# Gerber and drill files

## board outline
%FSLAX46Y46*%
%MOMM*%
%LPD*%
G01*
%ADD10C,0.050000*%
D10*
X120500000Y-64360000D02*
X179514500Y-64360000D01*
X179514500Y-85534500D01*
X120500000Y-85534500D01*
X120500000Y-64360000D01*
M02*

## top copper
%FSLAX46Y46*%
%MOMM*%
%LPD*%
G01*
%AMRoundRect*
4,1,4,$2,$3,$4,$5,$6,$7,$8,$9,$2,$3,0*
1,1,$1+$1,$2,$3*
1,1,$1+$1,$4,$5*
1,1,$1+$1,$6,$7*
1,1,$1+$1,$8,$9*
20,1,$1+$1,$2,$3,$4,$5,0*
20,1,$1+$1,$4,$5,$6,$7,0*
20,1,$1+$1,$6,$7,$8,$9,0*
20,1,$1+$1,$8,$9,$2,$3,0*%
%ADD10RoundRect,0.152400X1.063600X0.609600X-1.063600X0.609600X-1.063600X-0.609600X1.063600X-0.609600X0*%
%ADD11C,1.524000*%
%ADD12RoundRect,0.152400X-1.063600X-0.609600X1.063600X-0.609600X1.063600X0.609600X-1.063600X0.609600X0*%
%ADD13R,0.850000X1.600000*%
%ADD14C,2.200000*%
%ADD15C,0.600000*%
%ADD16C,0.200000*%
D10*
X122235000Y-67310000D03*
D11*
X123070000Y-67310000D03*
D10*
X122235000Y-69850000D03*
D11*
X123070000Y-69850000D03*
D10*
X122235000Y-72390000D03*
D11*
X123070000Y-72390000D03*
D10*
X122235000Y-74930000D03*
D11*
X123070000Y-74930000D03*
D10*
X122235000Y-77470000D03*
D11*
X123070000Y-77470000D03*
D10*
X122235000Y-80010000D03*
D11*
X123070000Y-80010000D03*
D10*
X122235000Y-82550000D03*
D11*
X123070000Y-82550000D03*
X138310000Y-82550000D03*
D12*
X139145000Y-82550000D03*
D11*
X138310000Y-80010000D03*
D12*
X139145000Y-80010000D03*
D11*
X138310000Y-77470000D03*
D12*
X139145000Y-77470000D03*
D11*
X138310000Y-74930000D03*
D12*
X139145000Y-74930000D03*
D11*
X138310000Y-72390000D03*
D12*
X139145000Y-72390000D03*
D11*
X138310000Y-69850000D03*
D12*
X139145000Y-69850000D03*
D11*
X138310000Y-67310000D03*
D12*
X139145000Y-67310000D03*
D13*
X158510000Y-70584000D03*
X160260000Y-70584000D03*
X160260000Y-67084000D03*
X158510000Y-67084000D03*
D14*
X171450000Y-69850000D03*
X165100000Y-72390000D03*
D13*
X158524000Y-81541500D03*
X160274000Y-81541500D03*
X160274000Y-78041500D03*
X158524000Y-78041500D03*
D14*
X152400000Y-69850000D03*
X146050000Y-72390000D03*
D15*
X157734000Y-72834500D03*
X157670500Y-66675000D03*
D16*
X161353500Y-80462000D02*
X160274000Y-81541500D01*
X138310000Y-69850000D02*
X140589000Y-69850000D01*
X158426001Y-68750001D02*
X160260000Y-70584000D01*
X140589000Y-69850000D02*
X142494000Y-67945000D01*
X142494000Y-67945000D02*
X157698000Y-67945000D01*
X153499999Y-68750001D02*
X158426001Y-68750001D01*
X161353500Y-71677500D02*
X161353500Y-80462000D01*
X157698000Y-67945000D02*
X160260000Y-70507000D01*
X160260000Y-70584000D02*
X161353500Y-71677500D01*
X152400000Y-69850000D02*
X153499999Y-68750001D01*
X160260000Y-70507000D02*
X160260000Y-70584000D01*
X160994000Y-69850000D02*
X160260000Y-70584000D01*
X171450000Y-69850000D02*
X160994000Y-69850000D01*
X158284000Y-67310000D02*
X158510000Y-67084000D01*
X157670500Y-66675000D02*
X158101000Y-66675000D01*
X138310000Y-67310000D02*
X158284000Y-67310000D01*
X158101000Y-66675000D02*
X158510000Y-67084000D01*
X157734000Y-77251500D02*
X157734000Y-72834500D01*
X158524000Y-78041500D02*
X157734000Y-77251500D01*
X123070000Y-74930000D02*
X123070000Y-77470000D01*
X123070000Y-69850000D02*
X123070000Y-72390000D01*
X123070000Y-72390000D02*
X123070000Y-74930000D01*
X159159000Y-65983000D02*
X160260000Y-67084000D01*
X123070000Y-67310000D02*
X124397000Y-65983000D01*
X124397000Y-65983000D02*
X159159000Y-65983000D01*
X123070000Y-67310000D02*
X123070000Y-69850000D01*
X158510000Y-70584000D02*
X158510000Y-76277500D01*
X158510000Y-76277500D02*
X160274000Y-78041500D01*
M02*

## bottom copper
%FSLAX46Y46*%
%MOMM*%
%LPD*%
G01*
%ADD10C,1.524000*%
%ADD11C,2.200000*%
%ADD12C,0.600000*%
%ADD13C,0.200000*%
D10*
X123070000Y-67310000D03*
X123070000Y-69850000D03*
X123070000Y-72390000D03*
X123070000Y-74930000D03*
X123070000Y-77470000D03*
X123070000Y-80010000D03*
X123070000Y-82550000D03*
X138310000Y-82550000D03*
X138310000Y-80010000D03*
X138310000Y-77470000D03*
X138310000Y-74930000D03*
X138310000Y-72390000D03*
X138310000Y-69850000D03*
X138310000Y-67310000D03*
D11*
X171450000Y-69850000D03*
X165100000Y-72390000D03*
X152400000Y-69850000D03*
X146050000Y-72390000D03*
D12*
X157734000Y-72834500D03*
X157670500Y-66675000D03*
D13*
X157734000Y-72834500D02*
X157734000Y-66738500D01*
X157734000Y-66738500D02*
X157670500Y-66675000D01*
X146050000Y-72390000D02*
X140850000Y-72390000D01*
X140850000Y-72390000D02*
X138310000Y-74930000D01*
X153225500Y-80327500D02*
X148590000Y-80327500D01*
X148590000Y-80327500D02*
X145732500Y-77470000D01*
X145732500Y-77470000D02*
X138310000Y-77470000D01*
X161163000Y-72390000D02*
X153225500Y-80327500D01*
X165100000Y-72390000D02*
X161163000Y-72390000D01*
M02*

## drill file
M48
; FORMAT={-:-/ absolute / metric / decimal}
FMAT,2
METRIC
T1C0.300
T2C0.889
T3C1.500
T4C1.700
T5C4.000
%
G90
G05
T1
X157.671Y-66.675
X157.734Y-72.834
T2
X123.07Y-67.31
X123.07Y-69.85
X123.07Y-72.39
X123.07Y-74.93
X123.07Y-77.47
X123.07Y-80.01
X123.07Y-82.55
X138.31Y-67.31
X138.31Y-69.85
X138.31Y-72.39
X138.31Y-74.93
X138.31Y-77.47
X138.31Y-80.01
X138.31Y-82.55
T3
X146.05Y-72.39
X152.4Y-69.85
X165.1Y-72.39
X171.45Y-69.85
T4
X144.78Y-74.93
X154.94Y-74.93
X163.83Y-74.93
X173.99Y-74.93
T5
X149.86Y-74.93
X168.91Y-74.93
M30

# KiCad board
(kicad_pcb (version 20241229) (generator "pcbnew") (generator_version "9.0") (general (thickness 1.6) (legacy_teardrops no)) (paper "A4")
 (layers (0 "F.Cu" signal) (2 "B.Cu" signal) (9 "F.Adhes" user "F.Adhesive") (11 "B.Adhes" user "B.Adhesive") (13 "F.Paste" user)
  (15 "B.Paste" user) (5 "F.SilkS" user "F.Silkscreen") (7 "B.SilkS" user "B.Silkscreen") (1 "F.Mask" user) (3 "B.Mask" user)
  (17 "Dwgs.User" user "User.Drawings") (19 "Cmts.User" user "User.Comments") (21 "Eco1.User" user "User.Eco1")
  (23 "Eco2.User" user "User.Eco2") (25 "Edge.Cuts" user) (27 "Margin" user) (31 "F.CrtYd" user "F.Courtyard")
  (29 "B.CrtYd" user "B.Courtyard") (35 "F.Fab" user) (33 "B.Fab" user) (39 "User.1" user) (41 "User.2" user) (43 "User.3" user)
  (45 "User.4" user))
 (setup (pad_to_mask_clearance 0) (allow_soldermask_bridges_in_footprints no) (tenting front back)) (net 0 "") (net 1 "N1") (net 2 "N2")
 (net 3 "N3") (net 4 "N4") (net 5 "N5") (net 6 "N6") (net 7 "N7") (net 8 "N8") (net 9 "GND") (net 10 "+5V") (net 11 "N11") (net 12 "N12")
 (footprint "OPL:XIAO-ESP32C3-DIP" (layer "F.Cu") (at 130.81 74.93)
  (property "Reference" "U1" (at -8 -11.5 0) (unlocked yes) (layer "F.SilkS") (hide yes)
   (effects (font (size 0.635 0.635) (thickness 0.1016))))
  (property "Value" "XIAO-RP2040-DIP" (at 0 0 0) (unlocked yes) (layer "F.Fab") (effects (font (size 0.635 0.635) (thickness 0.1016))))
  (pad "1" smd roundrect (at -8.575 -7.62 180) (size 2.432 1.524) (layers "F.Cu" "F.Mask") (roundrect_rratio 0.1) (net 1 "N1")
   (thermal_bridge_angle 45))
  (pad "1" thru_hole circle (at -7.74 -7.62 180) (size 1.524 1.524) (drill 0.889) (layers "*.Cu" "*.Mask") (remove_unused_layers no)
   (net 1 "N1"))
  (pad "2" smd roundrect (at -8.575 -5.08 180) (size 2.432 1.524) (layers "F.Cu" "F.Mask") (roundrect_rratio 0.1) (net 1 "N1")
   (thermal_bridge_angle 45))
  (pad "2" thru_hole circle (at -7.74 -5.08 180) (size 1.524 1.524) (drill 0.889) (layers "*.Cu" "*.Mask") (remove_unused_layers no)
   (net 1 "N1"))
  (pad "3" smd roundrect (at -8.575 -2.54 180) (size 2.432 1.524) (layers "F.Cu" "F.Mask") (roundrect_rratio 0.1) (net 1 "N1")
   (thermal_bridge_angle 45))
  (pad "3" thru_hole circle (at -7.74 -2.54 180) (size 1.524 1.524) (drill 0.889) (layers "*.Cu" "*.Mask") (remove_unused_layers no)
   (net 1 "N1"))
  (pad "4" smd roundrect (at -8.575 0 180) (size 2.432 1.524) (layers "F.Cu" "F.Mask") (roundrect_rratio 0.1) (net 1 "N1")
   (thermal_bridge_angle 45))
  (pad "4" thru_hole circle (at -7.74 0 180) (size 1.524 1.524) (drill 0.889) (layers "*.Cu" "*.Mask") (remove_unused_layers no)
   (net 1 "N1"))
  (pad "5" smd roundrect (at -8.575 2.54 180) (size 2.432 1.524) (layers "F.Cu" "F.Mask") (roundrect_rratio 0.1) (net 1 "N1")
   (thermal_bridge_angle 45))
  (pad "5" thru_hole circle (at -7.74 2.54 180) (size 1.524 1.524) (drill 0.889) (layers "*.Cu" "*.Mask") (remove_unused_layers no)
   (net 1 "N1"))
  (pad "6" smd roundrect (at -8.575 5.08 180) (size 2.432 1.524) (layers "F.Cu" "F.Mask") (roundrect_rratio 0.1) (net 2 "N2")
   (thermal_bridge_angle 45))
  (pad "6" thru_hole circle (at -7.74 5.08 180) (size 1.524 1.524) (drill 0.889) (layers "*.Cu" "*.Mask") (remove_unused_layers no)
   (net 2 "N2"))
  (pad "7" smd roundrect (at -8.575 7.62 180) (size 2.432 1.524) (layers "F.Cu" "F.Mask") (roundrect_rratio 0.1) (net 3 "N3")
   (thermal_bridge_angle 45))
  (pad "7" thru_hole circle (at -7.74 7.62 180) (size 1.524 1.524) (drill 0.889) (layers "*.Cu" "*.Mask") (remove_unused_layers no)
   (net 3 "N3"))
  (pad "8" thru_hole circle (at 7.5 7.62) (size 1.524 1.524) (drill 0.889) (layers "*.Cu" "*.Mask") (remove_unused_layers no) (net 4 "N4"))
  (pad "8" smd roundrect (at 8.335 7.62) (size 2.432 1.524) (layers "F.Cu" "F.Mask") (roundrect_rratio 0.1) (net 4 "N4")
   (thermal_bridge_angle 45))
  (pad "9" thru_hole circle (at 7.5 5.08) (size 1.524 1.524) (drill 0.889) (layers "*.Cu" "*.Mask") (remove_unused_layers no) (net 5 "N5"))
  (pad "9" smd roundrect (at 8.335 5.08) (size 2.432 1.524) (layers "F.Cu" "F.Mask") (roundrect_rratio 0.1) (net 5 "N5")
   (thermal_bridge_angle 45))
  (pad "10" thru_hole circle (at 7.5 2.54) (size 1.524 1.524) (drill 0.889) (layers "*.Cu" "*.Mask") (remove_unused_layers no) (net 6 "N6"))
  (pad "10" smd roundrect (at 8.335 2.54) (size 2.432 1.524) (layers "F.Cu" "F.Mask") (roundrect_rratio 0.1) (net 6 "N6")
   (thermal_bridge_angle 45))
  (pad "11" thru_hole circle (at 7.5 0) (size 1.524 1.524) (drill 0.889) (layers "*.Cu" "*.Mask") (remove_unused_layers no) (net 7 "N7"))
  (pad "11" smd roundrect (at 8.335 0) (size 2.432 1.524) (layers "F.Cu" "F.Mask") (roundrect_rratio 0.1) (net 7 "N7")
   (thermal_bridge_angle 45))
  (pad "12" thru_hole circle (at 7.5 -2.54) (size 1.524 1.524) (drill 0.889) (layers "*.Cu" "*.Mask") (remove_unused_layers no) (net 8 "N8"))
  (pad "12" smd roundrect (at 8.335 -2.54) (size 2.432 1.524) (layers "F.Cu" "F.Mask") (roundrect_rratio 0.1) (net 8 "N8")
   (thermal_bridge_angle 45))
  (pad "13" thru_hole circle (at 7.5 -5.08) (size 1.524 1.524) (drill 0.889) (layers "*.Cu" "*.Mask") (remove_unused_layers no)
   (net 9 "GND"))
  (pad "13" smd roundrect (at 8.335 -5.08) (size 2.432 1.524) (layers "F.Cu" "F.Mask") (roundrect_rratio 0.1) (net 9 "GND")
   (thermal_bridge_angle 45))
  (pad "14" thru_hole circle (at 7.5 -7.62) (size 1.524 1.524) (drill 0.889) (layers "*.Cu" "*.Mask") (remove_unused_layers no)
   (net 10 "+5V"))
  (pad "14" smd roundrect (at 8.335 -7.62) (size 2.432 1.524) (layers "F.Cu" "F.Mask") (roundrect_rratio 0.1) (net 10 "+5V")
   (thermal_bridge_angle 45)))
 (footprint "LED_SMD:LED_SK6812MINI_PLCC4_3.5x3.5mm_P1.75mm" (layer "F.Cu") (at 159.385 68.834 90)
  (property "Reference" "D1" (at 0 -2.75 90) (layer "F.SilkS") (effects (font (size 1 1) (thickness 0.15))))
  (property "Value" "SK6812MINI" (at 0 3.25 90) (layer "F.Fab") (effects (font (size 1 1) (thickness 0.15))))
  (pad "1" smd rect (at -1.75 -0.875 90) (size 1.6 0.85) (layers "F.Cu" "F.Mask" "F.Paste") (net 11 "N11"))
  (pad "2" smd rect (at -1.75 0.875 90) (size 1.6 0.85) (layers "F.Cu" "F.Mask" "F.Paste") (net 9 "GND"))
  (pad "3" smd rect (at 1.75 0.875 90) (size 1.6 0.85) (layers "F.Cu" "F.Mask" "F.Paste") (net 1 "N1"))
  (pad "4" smd rect (at 1.75 -0.875 90) (size 1.6 0.85) (layers "F.Cu" "F.Mask" "F.Paste") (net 10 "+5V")))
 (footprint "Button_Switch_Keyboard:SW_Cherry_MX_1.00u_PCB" (layer "F.Cu") (at 171.45 69.85)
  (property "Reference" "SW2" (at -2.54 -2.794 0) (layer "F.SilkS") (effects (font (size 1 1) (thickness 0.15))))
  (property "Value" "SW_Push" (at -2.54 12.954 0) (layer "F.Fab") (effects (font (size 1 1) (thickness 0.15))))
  (pad "" np_thru_hole circle (at -7.62 5.08) (size 1.7 1.7) (drill 1.7) (layers "*.Cu" "*.Mask"))
  (pad "" np_thru_hole circle (at -2.54 5.08) (size 4 4) (drill 4) (layers "*.Cu" "*.Mask"))
  (pad "" np_thru_hole circle (at 2.54 5.08) (size 1.7 1.7) (drill 1.7) (layers "*.Cu" "*.Mask"))
  (pad "1" thru_hole circle (at 0 0) (size 2.2 2.2) (drill 1.5) (layers "*.Cu" "*.Mask") (remove_unused_layers no) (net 9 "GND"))
  (pad "2" thru_hole circle (at -6.35 2.54) (size 2.2 2.2) (drill 1.5) (layers "*.Cu" "*.Mask") (remove_unused_layers no) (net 6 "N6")))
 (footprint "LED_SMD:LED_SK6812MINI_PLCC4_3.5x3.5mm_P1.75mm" (layer "F.Cu") (at 159.399 79.7915 90)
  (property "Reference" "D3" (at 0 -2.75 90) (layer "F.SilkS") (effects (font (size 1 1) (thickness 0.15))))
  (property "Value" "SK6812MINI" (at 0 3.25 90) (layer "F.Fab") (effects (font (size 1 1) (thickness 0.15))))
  (pad "1" smd rect (at -1.75 -0.875 90) (size 1.6 0.85) (layers "F.Cu" "F.Mask" "F.Paste") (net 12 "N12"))
  (pad "2" smd rect (at -1.75 0.875 90) (size 1.6 0.85) (layers "F.Cu" "F.Mask" "F.Paste") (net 9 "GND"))
  (pad "3" smd rect (at 1.75 0.875 90) (size 1.6 0.85) (layers "F.Cu" "F.Mask" "F.Paste") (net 11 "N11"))
  (pad "4" smd rect (at 1.75 -0.875 90) (size 1.6 0.85) (layers "F.Cu" "F.Mask" "F.Paste") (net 10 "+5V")))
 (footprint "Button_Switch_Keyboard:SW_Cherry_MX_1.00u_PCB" (layer "F.Cu") (at 152.4 69.85)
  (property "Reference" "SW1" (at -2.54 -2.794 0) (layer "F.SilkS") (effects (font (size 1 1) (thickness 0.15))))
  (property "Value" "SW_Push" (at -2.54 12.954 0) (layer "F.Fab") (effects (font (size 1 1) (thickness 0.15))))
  (pad "" np_thru_hole circle (at -7.62 5.08) (size 1.7 1.7) (drill 1.7) (layers "*.Cu" "*.Mask"))
  (pad "" np_thru_hole circle (at -2.54 5.08) (size 4 4) (drill 4) (layers "*.Cu" "*.Mask"))
  (pad "" np_thru_hole circle (at 2.54 5.08) (size 1.7 1.7) (drill 1.7) (layers "*.Cu" "*.Mask"))
  (pad "1" thru_hole circle (at 0 0) (size 2.2 2.2) (drill 1.5) (layers "*.Cu" "*.Mask") (remove_unused_layers no) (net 9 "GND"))
  (pad "2" thru_hole circle (at -6.35 2.54) (size 2.2 2.2) (drill 1.5) (layers "*.Cu" "*.Mask") (remove_unused_layers no) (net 7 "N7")))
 (gr_rect (start 120.5 64.36) (end 179.5145 85.5345) (stroke (width 0.05) (type default)) (fill no) (layer "Edge.Cuts"))
 (segment (start 161.3535 80.462) (end 160.274 81.5415) (width 0.2) (layer "F.Cu") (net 9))
 (segment (start 138.31 69.85) (end 140.589 69.85) (width 0.2) (layer "F.Cu") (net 9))
 (segment (start 158.426001 68.750001) (end 160.26 70.584) (width 0.2) (layer "F.Cu") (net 9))
 (segment (start 140.589 69.85) (end 142.494 67.945) (width 0.2) (layer "F.Cu") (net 9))
 (segment (start 142.494 67.945) (end 157.698 67.945) (width 0.2) (layer "F.Cu") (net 9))
 (segment (start 153.499999 68.750001) (end 158.426001 68.750001) (width 0.2) (layer "F.Cu") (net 9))
 (segment (start 161.3535 71.6775) (end 161.3535 80.462) (width 0.2) (layer "F.Cu") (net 9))
 (segment (start 157.698 67.945) (end 160.26 70.507) (width 0.2) (layer "F.Cu") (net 9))
 (segment (start 160.26 70.584) (end 161.3535 71.6775) (width 0.2) (layer "F.Cu") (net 9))
 (segment (start 152.4 69.85) (end 153.499999 68.750001) (width 0.2) (layer "F.Cu") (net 9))
 (segment (start 160.26 70.507) (end 160.26 70.584) (width 0.2) (layer "F.Cu") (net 9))
 (segment (start 160.994 69.85) (end 160.26 70.584) (width 0.2) (layer "F.Cu") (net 9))
 (segment (start 171.45 69.85) (end 160.994 69.85) (width 0.2) (layer "F.Cu") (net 9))
 (segment (start 158.284 67.31) (end 158.51 67.084) (width 0.2) (layer "F.Cu") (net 10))
 (segment (start 157.6705 66.675) (end 158.101 66.675) (width 0.2) (layer "F.Cu") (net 10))
 (segment (start 138.31 67.31) (end 158.284 67.31) (width 0.2) (layer "F.Cu") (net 10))
 (segment (start 158.101 66.675) (end 158.51 67.084) (width 0.2) (layer "F.Cu") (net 10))
 (segment (start 157.734 77.2515) (end 157.734 72.8345) (width 0.2) (layer "F.Cu") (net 10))
 (segment (start 158.524 78.0415) (end 157.734 77.2515) (width 0.2) (layer "F.Cu") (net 10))
 (via (at 157.734 72.8345) (size 0.6) (drill 0.3) (layers "F.Cu" "B.Cu") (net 10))
 (via (at 157.6705 66.675) (size 0.6) (drill 0.3) (layers "F.Cu" "B.Cu") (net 10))
 (segment (start 157.734 72.8345) (end 157.734 66.7385) (width 0.2) (layer "B.Cu") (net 10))
 (segment (start 157.734 66.7385) (end 157.6705 66.675) (width 0.2) (layer "B.Cu") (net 10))
 (segment (start 123.07 74.93) (end 123.07 77.47) (width 0.2) (layer "F.Cu") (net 1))
 (segment (start 123.07 69.85) (end 123.07 72.39) (width 0.2) (layer "F.Cu") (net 1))
 (segment (start 123.07 72.39) (end 123.07 74.93) (width 0.2) (layer "F.Cu") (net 1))
 (segment (start 159.159 65.983) (end 160.26 67.084) (width 0.2) (layer "F.Cu") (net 1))
 (segment (start 123.07 67.31) (end 124.397 65.983) (width 0.2) (layer "F.Cu") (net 1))
 (segment (start 124.397 65.983) (end 159.159 65.983) (width 0.2) (layer "F.Cu") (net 1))
 (segment (start 123.07 67.31) (end 123.07 69.85) (width 0.2) (layer "F.Cu") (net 1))
 (segment (start 146.05 72.39) (end 140.85 72.39) (width 0.2) (layer "B.Cu") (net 7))
 (segment (start 140.85 72.39) (end 138.31 74.93) (width 0.2) (layer "B.Cu") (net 7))
 (segment (start 153.2255 80.3275) (end 148.59 80.3275) (width 0.2) (layer "B.Cu") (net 6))
 (segment (start 148.59 80.3275) (end 145.7325 77.47) (width 0.2) (layer "B.Cu") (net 6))
 (segment (start 145.7325 77.47) (end 138.31 77.47) (width 0.2) (layer "B.Cu") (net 6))
 (segment (start 161.163 72.39) (end 153.2255 80.3275) (width 0.2) (layer "B.Cu") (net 6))
 (segment (start 165.1 72.39) (end 161.163 72.39) (width 0.2) (layer "B.Cu") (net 6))
 (segment (start 158.51 70.584) (end 158.51 76.2775) (width 0.2) (layer "F.Cu") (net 11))
 (segment (start 158.51 76.2775) (end 160.274 78.0415) (width 0.2) (layer "F.Cu") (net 11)))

